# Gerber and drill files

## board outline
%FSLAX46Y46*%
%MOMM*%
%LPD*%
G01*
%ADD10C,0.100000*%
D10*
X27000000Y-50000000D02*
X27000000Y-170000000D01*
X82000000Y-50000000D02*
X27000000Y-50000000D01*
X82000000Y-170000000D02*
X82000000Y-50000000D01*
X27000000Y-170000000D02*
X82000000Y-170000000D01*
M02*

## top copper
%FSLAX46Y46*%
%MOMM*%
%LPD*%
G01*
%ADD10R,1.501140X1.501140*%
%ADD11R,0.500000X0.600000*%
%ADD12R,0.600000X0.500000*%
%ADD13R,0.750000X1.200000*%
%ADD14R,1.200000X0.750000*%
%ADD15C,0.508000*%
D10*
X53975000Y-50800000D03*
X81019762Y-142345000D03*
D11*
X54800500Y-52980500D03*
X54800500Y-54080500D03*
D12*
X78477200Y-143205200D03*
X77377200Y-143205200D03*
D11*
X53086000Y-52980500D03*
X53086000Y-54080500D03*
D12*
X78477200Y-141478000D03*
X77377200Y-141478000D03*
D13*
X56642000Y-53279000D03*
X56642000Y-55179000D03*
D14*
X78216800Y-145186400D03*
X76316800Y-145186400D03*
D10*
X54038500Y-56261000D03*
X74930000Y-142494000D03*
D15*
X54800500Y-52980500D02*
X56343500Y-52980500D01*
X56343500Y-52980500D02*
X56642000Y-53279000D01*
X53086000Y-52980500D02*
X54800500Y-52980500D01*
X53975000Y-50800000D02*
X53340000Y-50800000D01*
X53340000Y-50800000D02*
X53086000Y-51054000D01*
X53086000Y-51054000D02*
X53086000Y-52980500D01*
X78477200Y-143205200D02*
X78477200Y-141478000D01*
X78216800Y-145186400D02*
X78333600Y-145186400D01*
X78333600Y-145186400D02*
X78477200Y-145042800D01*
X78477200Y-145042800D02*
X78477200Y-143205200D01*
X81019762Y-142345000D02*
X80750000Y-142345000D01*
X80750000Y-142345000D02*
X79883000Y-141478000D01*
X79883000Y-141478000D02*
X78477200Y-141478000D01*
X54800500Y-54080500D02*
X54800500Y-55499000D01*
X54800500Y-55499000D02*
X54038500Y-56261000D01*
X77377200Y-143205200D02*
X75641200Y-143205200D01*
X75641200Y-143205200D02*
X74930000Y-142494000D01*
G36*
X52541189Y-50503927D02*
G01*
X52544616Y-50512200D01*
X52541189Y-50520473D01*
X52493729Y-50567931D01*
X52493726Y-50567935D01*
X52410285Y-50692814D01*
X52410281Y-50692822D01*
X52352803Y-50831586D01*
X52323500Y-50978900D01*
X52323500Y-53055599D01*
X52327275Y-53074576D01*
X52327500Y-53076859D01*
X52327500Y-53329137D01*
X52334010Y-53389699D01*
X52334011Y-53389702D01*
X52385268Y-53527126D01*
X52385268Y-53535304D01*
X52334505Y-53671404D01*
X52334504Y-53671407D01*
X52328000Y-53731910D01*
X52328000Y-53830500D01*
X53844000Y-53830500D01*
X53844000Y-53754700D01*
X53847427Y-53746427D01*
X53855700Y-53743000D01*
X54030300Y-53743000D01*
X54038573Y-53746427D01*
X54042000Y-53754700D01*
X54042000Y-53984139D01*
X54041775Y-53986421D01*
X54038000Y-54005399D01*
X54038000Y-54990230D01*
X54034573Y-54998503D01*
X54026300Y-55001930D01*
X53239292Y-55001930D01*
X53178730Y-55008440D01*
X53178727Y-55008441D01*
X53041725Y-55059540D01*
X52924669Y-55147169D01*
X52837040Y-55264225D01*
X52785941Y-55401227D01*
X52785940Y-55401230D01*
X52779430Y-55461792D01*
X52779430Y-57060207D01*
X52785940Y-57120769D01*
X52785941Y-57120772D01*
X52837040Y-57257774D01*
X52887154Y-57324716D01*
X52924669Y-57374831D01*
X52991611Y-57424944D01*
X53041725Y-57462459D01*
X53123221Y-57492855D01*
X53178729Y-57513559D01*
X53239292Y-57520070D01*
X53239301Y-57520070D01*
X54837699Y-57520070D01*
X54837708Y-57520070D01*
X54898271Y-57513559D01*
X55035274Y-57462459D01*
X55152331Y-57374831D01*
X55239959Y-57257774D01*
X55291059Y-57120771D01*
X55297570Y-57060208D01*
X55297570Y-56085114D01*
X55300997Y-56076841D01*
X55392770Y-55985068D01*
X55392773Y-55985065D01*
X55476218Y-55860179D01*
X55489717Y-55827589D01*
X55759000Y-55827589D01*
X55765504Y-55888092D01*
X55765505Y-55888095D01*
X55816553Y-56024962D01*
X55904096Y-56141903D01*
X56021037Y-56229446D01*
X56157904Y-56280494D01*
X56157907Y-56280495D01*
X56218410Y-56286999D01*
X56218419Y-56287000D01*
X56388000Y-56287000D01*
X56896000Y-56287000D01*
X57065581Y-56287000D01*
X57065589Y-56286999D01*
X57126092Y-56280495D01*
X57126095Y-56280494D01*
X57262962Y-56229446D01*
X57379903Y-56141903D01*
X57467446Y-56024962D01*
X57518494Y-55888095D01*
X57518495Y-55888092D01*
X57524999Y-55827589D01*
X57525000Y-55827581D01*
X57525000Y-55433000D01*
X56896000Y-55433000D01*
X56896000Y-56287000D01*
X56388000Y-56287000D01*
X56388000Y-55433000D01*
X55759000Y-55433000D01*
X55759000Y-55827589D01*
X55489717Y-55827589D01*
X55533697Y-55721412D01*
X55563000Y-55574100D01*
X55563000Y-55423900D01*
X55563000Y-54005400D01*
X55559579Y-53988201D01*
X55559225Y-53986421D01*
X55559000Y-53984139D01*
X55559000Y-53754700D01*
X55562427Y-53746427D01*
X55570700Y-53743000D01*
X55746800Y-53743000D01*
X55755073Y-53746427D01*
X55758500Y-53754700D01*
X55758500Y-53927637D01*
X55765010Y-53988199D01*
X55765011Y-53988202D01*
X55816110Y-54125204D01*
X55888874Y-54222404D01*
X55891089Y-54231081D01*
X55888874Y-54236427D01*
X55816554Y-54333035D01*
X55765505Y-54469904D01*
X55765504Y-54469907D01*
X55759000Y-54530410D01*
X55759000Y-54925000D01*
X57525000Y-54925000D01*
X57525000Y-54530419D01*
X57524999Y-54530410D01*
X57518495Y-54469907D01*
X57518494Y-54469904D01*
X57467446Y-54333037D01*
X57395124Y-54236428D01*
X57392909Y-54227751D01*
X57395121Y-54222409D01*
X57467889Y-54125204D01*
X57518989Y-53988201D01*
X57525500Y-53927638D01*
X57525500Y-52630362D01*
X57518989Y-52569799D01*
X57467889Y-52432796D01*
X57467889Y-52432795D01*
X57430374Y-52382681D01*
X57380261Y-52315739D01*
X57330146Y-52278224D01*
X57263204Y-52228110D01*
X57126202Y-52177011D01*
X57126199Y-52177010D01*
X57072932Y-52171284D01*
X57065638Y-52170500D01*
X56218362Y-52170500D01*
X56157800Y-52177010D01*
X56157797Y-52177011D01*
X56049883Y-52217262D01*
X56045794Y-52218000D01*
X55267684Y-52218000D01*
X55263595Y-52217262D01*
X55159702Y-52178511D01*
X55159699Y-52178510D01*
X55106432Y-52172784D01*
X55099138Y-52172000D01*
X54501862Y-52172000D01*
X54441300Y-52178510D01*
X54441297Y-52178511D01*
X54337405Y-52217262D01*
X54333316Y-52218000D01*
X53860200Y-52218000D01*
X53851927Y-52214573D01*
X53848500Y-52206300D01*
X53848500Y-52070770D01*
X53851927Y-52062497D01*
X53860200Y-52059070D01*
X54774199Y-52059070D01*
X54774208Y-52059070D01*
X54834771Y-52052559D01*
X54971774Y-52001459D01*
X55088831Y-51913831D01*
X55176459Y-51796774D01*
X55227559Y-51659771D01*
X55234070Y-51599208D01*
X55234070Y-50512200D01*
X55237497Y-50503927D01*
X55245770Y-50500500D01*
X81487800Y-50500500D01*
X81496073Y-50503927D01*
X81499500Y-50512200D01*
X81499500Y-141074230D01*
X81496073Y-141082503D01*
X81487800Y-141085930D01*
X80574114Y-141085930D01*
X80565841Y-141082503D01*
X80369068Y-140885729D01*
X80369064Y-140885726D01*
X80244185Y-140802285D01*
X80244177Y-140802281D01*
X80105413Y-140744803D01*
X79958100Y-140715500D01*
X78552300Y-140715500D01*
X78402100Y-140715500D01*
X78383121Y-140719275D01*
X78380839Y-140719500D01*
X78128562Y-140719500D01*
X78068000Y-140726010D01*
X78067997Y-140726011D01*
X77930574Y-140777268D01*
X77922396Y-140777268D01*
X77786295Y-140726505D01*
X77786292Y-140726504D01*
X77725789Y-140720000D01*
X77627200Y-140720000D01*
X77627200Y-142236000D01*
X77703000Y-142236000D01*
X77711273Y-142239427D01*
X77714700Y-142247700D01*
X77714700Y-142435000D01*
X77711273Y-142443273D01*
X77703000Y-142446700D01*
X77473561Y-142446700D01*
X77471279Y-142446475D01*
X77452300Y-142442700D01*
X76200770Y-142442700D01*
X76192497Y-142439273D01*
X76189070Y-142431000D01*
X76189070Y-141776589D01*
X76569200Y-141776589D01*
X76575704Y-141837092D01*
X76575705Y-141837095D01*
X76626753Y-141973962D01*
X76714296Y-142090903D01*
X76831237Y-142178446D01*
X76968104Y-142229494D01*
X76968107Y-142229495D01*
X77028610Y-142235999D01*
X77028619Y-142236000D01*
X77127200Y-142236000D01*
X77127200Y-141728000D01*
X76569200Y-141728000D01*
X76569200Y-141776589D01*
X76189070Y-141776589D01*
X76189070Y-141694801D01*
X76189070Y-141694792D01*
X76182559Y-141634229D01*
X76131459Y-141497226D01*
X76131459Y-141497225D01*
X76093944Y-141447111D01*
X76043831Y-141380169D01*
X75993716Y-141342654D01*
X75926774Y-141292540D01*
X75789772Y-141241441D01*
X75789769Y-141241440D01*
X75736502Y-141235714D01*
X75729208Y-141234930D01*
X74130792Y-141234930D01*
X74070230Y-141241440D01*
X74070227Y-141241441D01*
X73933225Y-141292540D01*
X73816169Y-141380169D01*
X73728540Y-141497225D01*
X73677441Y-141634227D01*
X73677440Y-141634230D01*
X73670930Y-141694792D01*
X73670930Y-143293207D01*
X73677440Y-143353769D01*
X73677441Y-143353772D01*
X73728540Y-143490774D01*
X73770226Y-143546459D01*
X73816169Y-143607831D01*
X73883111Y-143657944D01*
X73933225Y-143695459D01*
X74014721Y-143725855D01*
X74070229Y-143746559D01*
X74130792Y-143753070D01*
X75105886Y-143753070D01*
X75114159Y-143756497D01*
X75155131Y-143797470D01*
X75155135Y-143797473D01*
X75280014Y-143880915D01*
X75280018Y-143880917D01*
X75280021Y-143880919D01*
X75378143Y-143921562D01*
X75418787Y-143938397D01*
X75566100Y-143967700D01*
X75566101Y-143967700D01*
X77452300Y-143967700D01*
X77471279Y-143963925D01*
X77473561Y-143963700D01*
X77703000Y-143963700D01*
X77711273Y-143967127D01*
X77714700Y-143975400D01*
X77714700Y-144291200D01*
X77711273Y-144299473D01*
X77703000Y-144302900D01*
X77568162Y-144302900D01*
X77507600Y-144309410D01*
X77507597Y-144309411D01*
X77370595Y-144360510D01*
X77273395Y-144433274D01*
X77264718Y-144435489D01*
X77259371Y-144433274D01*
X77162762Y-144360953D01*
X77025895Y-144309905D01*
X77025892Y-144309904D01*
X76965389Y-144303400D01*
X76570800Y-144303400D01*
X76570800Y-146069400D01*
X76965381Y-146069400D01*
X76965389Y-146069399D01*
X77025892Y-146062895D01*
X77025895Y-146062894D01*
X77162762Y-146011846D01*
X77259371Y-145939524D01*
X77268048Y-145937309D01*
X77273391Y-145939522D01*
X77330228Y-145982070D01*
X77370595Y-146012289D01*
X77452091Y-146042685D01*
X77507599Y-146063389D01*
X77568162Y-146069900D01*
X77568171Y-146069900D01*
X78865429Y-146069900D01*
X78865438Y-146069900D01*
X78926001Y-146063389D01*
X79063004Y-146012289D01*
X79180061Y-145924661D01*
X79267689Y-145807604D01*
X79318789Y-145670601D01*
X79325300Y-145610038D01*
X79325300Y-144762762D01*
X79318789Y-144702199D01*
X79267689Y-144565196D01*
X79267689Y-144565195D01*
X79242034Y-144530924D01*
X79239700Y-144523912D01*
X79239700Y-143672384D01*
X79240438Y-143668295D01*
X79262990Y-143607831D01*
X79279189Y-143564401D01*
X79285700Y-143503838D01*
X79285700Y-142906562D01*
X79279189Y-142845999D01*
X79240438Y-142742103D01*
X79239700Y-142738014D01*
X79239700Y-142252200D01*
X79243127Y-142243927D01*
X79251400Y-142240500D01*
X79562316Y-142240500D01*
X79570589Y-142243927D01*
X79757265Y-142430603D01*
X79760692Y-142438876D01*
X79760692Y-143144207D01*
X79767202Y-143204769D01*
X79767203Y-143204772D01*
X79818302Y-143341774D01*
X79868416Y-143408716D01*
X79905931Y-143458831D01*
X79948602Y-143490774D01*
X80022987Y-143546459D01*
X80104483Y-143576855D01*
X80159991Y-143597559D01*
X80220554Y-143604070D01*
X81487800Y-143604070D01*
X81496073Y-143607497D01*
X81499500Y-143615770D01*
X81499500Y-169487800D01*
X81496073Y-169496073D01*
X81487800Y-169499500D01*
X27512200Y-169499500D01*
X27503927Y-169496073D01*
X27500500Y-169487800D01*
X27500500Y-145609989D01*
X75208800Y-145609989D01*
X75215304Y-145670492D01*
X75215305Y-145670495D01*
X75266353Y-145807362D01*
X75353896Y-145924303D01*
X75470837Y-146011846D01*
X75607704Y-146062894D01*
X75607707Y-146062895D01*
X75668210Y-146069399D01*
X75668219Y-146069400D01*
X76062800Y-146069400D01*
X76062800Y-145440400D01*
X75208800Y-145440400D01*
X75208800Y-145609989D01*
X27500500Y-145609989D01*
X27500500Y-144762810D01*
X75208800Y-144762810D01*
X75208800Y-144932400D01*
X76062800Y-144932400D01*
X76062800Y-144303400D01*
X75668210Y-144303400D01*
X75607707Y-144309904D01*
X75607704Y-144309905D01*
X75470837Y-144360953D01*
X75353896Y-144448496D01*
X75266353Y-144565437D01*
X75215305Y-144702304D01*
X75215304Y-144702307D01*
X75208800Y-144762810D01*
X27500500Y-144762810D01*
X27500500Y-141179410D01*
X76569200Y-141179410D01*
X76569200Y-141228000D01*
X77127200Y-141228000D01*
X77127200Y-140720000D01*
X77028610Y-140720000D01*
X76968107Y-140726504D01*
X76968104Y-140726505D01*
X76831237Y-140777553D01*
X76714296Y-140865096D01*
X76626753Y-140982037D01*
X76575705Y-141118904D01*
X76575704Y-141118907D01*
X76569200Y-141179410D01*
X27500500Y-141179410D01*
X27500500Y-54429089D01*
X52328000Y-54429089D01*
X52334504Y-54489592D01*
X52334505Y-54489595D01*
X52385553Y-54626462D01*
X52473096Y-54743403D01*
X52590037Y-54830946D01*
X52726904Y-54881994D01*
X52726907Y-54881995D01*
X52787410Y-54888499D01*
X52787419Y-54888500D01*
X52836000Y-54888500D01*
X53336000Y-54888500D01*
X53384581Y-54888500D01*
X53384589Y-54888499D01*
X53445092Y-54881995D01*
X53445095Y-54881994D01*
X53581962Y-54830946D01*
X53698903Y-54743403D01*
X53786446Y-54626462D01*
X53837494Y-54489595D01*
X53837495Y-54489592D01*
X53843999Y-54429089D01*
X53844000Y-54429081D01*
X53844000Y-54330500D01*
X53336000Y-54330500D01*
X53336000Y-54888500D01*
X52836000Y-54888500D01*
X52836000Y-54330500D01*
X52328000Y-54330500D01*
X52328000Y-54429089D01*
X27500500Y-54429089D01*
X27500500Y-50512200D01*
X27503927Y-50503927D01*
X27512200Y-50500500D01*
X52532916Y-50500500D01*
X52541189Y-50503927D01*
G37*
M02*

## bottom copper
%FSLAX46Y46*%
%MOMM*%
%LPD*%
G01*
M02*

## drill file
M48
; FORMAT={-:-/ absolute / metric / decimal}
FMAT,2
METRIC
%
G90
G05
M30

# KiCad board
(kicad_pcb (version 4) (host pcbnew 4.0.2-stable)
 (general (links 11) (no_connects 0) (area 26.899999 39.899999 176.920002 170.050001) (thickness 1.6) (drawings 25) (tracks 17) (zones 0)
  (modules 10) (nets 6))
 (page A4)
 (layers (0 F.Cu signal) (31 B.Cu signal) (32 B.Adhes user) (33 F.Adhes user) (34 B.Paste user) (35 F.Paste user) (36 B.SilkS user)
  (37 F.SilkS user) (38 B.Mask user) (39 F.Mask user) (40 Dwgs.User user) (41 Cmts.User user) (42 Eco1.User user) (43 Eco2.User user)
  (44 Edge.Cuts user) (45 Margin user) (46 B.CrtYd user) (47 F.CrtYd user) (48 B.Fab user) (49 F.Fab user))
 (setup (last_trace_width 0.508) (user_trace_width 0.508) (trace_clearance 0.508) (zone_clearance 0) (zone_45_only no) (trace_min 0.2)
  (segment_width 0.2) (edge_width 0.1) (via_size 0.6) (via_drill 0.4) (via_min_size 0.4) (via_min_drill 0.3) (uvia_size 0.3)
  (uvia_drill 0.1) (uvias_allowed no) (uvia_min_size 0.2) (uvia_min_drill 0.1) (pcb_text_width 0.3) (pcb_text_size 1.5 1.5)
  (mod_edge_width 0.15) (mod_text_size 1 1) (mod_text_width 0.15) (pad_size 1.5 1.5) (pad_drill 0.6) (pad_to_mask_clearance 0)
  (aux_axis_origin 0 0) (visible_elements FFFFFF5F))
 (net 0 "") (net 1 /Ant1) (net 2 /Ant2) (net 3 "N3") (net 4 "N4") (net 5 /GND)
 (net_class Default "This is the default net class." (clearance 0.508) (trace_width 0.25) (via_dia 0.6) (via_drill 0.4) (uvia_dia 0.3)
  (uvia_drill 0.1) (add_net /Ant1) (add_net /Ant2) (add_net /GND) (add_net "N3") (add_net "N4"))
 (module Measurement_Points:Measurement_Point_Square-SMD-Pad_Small (layer F.Cu) (at 53.975 50.8)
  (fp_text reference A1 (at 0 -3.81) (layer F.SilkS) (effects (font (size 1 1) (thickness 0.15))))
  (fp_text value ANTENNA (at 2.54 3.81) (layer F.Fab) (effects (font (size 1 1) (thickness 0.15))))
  (pad 1 smd rect (at 0 0) (size 1.50114 1.50114) (layers F.Cu F.Mask) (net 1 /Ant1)))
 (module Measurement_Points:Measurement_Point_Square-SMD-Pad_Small (layer F.Cu) (at 81.019762 142.345)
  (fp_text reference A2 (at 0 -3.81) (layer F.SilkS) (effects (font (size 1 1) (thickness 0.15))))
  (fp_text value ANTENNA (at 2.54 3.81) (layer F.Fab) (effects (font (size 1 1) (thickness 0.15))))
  (pad 1 smd rect (at 0 0) (size 1.50114 1.50114) (layers F.Cu F.Mask) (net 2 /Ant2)))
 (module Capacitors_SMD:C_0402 (layer F.Cu) (at 54.8005 53.5305 270)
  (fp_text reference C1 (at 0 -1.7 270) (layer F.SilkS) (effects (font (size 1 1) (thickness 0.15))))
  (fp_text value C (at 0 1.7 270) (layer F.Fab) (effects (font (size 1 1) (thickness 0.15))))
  (pad 1 smd rect (at -0.55 0 270) (size 0.6 0.5) (layers F.Cu F.Paste F.Mask) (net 1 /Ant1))
  (pad 2 smd rect (at 0.55 0 270) (size 0.6 0.5) (layers F.Cu F.Paste F.Mask) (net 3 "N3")))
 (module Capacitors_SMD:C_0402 (layer F.Cu) (at 77.9272 143.2052 180)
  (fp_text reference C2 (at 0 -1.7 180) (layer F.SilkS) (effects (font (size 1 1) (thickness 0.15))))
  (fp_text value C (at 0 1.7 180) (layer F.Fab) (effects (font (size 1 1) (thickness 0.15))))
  (pad 1 smd rect (at -0.55 0 180) (size 0.6 0.5) (layers F.Cu F.Paste F.Mask) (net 2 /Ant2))
  (pad 2 smd rect (at 0.55 0 180) (size 0.6 0.5) (layers F.Cu F.Paste F.Mask) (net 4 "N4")))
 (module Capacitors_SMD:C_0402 (layer F.Cu) (at 53.086 53.5305 270)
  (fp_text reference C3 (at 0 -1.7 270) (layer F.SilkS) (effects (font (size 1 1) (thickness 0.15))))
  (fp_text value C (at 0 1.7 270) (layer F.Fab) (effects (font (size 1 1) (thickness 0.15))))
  (pad 1 smd rect (at -0.55 0 270) (size 0.6 0.5) (layers F.Cu F.Paste F.Mask) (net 1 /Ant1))
  (pad 2 smd rect (at 0.55 0 270) (size 0.6 0.5) (layers F.Cu F.Paste F.Mask) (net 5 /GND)))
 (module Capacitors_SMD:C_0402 (layer F.Cu) (at 77.9272 141.478 180)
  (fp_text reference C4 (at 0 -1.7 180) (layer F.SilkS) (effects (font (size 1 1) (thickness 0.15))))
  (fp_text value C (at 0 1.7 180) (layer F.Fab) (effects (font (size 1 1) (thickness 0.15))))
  (pad 1 smd rect (at -0.55 0 180) (size 0.6 0.5) (layers F.Cu F.Paste F.Mask) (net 2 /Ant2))
  (pad 2 smd rect (at 0.55 0 180) (size 0.6 0.5) (layers F.Cu F.Paste F.Mask) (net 5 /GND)))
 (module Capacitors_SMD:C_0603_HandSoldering (layer F.Cu) (at 56.642 54.229 270)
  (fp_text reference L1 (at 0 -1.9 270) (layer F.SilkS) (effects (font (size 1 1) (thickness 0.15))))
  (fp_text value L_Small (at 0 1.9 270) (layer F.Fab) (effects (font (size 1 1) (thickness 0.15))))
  (pad 1 smd rect (at -0.95 0 270) (size 1.2 0.75) (layers F.Cu F.Paste F.Mask) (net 1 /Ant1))
  (pad 2 smd rect (at 0.95 0 270) (size 1.2 0.75) (layers F.Cu F.Paste F.Mask) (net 5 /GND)))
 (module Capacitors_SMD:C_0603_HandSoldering (layer F.Cu) (at 77.2668 145.1864 180)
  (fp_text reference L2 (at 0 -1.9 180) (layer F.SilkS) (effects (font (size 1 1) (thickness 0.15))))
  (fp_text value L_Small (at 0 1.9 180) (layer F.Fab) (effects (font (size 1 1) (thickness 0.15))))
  (pad 1 smd rect (at -0.95 0 180) (size 1.2 0.75) (layers F.Cu F.Paste F.Mask) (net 2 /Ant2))
  (pad 2 smd rect (at 0.95 0 180) (size 1.2 0.75) (layers F.Cu F.Paste F.Mask) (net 5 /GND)))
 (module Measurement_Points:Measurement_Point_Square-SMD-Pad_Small (layer F.Cu) (at 54.0385 56.261)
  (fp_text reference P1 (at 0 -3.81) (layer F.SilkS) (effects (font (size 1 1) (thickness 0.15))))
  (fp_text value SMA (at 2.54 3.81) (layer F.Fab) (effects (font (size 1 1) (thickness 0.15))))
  (pad 1 smd rect (at 0 0) (size 1.50114 1.50114) (layers F.Cu F.Mask) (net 3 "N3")))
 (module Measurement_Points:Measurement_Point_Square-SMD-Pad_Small (layer F.Cu) (at 74.93 142.494)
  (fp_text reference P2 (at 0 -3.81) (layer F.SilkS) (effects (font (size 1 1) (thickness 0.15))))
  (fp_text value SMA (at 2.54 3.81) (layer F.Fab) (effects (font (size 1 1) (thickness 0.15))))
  (pad 1 smd rect (at 0 0) (size 1.50114 1.50114) (layers F.Cu F.Mask) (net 4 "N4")))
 (gr_line (start 27 50) (end 27 170) (angle 90) (layer Edge.Cuts) (width 0.1))
 (gr_line (start 82 50) (end 27 50) (angle 90) (layer Edge.Cuts) (width 0.1))
 (gr_line (start 82 170) (end 82 50) (angle 90) (layer Edge.Cuts) (width 0.1))
 (gr_line (start 27 170) (end 82 170) (angle 90) (layer Edge.Cuts) (width 0.1))
 (segment (start 54.8005 52.9805) (end 56.3435 52.9805) (width 0.508) (layer F.Cu) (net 1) (status C00000))
 (segment (start 56.3435 52.9805) (end 56.642 53.279) (width 0.508) (layer F.Cu) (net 1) (status C00000))
 (segment (start 53.086 52.9805) (end 54.8005 52.9805) (width 0.508) (layer F.Cu) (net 1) (status C00000))
 (segment (start 53.975 50.8) (end 53.34 50.8) (width 0.508) (layer F.Cu) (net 1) (status C00000))
 (segment (start 53.34 50.8) (end 53.086 51.054) (width 0.508) (layer F.Cu) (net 1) (status 400000))
 (segment (start 53.086 51.054) (end 53.086 52.9805) (width 0.508) (layer F.Cu) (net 1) (status 800000))
 (segment (start 78.4772 143.2052) (end 78.4772 141.478) (width 0.508) (layer F.Cu) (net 2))
 (segment (start 78.2168 145.1864) (end 78.3336 145.1864) (width 0.508) (layer F.Cu) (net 2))
 (segment (start 78.3336 145.1864) (end 78.4772 145.0428) (width 0.508) (layer F.Cu) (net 2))
 (segment (start 78.4772 145.0428) (end 78.4772 143.2052) (width 0.508) (layer F.Cu) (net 2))
 (segment (start 81.019762 142.345) (end 80.75 142.345) (width 0.508) (layer F.Cu) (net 2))
 (segment (start 80.75 142.345) (end 79.883 141.478) (width 0.508) (layer F.Cu) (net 2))
 (segment (start 79.883 141.478) (end 78.4772 141.478) (width 0.508) (layer F.Cu) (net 2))
 (segment (start 54.8005 54.0805) (end 54.8005 55.499) (width 0.508) (layer F.Cu) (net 3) (status 400000))
 (segment (start 54.8005 55.499) (end 54.0385 56.261) (width 0.508) (layer F.Cu) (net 3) (status 800000))
 (segment (start 77.3772 143.2052) (end 75.6412 143.2052) (width 0.508) (layer F.Cu) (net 4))
 (segment (start 75.6412 143.2052) (end 74.93 142.494) (width 0.508) (layer F.Cu) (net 4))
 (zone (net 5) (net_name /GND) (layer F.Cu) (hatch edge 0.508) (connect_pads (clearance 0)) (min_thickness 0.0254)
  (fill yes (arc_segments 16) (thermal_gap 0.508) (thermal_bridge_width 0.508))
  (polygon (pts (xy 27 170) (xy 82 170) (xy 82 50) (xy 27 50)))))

